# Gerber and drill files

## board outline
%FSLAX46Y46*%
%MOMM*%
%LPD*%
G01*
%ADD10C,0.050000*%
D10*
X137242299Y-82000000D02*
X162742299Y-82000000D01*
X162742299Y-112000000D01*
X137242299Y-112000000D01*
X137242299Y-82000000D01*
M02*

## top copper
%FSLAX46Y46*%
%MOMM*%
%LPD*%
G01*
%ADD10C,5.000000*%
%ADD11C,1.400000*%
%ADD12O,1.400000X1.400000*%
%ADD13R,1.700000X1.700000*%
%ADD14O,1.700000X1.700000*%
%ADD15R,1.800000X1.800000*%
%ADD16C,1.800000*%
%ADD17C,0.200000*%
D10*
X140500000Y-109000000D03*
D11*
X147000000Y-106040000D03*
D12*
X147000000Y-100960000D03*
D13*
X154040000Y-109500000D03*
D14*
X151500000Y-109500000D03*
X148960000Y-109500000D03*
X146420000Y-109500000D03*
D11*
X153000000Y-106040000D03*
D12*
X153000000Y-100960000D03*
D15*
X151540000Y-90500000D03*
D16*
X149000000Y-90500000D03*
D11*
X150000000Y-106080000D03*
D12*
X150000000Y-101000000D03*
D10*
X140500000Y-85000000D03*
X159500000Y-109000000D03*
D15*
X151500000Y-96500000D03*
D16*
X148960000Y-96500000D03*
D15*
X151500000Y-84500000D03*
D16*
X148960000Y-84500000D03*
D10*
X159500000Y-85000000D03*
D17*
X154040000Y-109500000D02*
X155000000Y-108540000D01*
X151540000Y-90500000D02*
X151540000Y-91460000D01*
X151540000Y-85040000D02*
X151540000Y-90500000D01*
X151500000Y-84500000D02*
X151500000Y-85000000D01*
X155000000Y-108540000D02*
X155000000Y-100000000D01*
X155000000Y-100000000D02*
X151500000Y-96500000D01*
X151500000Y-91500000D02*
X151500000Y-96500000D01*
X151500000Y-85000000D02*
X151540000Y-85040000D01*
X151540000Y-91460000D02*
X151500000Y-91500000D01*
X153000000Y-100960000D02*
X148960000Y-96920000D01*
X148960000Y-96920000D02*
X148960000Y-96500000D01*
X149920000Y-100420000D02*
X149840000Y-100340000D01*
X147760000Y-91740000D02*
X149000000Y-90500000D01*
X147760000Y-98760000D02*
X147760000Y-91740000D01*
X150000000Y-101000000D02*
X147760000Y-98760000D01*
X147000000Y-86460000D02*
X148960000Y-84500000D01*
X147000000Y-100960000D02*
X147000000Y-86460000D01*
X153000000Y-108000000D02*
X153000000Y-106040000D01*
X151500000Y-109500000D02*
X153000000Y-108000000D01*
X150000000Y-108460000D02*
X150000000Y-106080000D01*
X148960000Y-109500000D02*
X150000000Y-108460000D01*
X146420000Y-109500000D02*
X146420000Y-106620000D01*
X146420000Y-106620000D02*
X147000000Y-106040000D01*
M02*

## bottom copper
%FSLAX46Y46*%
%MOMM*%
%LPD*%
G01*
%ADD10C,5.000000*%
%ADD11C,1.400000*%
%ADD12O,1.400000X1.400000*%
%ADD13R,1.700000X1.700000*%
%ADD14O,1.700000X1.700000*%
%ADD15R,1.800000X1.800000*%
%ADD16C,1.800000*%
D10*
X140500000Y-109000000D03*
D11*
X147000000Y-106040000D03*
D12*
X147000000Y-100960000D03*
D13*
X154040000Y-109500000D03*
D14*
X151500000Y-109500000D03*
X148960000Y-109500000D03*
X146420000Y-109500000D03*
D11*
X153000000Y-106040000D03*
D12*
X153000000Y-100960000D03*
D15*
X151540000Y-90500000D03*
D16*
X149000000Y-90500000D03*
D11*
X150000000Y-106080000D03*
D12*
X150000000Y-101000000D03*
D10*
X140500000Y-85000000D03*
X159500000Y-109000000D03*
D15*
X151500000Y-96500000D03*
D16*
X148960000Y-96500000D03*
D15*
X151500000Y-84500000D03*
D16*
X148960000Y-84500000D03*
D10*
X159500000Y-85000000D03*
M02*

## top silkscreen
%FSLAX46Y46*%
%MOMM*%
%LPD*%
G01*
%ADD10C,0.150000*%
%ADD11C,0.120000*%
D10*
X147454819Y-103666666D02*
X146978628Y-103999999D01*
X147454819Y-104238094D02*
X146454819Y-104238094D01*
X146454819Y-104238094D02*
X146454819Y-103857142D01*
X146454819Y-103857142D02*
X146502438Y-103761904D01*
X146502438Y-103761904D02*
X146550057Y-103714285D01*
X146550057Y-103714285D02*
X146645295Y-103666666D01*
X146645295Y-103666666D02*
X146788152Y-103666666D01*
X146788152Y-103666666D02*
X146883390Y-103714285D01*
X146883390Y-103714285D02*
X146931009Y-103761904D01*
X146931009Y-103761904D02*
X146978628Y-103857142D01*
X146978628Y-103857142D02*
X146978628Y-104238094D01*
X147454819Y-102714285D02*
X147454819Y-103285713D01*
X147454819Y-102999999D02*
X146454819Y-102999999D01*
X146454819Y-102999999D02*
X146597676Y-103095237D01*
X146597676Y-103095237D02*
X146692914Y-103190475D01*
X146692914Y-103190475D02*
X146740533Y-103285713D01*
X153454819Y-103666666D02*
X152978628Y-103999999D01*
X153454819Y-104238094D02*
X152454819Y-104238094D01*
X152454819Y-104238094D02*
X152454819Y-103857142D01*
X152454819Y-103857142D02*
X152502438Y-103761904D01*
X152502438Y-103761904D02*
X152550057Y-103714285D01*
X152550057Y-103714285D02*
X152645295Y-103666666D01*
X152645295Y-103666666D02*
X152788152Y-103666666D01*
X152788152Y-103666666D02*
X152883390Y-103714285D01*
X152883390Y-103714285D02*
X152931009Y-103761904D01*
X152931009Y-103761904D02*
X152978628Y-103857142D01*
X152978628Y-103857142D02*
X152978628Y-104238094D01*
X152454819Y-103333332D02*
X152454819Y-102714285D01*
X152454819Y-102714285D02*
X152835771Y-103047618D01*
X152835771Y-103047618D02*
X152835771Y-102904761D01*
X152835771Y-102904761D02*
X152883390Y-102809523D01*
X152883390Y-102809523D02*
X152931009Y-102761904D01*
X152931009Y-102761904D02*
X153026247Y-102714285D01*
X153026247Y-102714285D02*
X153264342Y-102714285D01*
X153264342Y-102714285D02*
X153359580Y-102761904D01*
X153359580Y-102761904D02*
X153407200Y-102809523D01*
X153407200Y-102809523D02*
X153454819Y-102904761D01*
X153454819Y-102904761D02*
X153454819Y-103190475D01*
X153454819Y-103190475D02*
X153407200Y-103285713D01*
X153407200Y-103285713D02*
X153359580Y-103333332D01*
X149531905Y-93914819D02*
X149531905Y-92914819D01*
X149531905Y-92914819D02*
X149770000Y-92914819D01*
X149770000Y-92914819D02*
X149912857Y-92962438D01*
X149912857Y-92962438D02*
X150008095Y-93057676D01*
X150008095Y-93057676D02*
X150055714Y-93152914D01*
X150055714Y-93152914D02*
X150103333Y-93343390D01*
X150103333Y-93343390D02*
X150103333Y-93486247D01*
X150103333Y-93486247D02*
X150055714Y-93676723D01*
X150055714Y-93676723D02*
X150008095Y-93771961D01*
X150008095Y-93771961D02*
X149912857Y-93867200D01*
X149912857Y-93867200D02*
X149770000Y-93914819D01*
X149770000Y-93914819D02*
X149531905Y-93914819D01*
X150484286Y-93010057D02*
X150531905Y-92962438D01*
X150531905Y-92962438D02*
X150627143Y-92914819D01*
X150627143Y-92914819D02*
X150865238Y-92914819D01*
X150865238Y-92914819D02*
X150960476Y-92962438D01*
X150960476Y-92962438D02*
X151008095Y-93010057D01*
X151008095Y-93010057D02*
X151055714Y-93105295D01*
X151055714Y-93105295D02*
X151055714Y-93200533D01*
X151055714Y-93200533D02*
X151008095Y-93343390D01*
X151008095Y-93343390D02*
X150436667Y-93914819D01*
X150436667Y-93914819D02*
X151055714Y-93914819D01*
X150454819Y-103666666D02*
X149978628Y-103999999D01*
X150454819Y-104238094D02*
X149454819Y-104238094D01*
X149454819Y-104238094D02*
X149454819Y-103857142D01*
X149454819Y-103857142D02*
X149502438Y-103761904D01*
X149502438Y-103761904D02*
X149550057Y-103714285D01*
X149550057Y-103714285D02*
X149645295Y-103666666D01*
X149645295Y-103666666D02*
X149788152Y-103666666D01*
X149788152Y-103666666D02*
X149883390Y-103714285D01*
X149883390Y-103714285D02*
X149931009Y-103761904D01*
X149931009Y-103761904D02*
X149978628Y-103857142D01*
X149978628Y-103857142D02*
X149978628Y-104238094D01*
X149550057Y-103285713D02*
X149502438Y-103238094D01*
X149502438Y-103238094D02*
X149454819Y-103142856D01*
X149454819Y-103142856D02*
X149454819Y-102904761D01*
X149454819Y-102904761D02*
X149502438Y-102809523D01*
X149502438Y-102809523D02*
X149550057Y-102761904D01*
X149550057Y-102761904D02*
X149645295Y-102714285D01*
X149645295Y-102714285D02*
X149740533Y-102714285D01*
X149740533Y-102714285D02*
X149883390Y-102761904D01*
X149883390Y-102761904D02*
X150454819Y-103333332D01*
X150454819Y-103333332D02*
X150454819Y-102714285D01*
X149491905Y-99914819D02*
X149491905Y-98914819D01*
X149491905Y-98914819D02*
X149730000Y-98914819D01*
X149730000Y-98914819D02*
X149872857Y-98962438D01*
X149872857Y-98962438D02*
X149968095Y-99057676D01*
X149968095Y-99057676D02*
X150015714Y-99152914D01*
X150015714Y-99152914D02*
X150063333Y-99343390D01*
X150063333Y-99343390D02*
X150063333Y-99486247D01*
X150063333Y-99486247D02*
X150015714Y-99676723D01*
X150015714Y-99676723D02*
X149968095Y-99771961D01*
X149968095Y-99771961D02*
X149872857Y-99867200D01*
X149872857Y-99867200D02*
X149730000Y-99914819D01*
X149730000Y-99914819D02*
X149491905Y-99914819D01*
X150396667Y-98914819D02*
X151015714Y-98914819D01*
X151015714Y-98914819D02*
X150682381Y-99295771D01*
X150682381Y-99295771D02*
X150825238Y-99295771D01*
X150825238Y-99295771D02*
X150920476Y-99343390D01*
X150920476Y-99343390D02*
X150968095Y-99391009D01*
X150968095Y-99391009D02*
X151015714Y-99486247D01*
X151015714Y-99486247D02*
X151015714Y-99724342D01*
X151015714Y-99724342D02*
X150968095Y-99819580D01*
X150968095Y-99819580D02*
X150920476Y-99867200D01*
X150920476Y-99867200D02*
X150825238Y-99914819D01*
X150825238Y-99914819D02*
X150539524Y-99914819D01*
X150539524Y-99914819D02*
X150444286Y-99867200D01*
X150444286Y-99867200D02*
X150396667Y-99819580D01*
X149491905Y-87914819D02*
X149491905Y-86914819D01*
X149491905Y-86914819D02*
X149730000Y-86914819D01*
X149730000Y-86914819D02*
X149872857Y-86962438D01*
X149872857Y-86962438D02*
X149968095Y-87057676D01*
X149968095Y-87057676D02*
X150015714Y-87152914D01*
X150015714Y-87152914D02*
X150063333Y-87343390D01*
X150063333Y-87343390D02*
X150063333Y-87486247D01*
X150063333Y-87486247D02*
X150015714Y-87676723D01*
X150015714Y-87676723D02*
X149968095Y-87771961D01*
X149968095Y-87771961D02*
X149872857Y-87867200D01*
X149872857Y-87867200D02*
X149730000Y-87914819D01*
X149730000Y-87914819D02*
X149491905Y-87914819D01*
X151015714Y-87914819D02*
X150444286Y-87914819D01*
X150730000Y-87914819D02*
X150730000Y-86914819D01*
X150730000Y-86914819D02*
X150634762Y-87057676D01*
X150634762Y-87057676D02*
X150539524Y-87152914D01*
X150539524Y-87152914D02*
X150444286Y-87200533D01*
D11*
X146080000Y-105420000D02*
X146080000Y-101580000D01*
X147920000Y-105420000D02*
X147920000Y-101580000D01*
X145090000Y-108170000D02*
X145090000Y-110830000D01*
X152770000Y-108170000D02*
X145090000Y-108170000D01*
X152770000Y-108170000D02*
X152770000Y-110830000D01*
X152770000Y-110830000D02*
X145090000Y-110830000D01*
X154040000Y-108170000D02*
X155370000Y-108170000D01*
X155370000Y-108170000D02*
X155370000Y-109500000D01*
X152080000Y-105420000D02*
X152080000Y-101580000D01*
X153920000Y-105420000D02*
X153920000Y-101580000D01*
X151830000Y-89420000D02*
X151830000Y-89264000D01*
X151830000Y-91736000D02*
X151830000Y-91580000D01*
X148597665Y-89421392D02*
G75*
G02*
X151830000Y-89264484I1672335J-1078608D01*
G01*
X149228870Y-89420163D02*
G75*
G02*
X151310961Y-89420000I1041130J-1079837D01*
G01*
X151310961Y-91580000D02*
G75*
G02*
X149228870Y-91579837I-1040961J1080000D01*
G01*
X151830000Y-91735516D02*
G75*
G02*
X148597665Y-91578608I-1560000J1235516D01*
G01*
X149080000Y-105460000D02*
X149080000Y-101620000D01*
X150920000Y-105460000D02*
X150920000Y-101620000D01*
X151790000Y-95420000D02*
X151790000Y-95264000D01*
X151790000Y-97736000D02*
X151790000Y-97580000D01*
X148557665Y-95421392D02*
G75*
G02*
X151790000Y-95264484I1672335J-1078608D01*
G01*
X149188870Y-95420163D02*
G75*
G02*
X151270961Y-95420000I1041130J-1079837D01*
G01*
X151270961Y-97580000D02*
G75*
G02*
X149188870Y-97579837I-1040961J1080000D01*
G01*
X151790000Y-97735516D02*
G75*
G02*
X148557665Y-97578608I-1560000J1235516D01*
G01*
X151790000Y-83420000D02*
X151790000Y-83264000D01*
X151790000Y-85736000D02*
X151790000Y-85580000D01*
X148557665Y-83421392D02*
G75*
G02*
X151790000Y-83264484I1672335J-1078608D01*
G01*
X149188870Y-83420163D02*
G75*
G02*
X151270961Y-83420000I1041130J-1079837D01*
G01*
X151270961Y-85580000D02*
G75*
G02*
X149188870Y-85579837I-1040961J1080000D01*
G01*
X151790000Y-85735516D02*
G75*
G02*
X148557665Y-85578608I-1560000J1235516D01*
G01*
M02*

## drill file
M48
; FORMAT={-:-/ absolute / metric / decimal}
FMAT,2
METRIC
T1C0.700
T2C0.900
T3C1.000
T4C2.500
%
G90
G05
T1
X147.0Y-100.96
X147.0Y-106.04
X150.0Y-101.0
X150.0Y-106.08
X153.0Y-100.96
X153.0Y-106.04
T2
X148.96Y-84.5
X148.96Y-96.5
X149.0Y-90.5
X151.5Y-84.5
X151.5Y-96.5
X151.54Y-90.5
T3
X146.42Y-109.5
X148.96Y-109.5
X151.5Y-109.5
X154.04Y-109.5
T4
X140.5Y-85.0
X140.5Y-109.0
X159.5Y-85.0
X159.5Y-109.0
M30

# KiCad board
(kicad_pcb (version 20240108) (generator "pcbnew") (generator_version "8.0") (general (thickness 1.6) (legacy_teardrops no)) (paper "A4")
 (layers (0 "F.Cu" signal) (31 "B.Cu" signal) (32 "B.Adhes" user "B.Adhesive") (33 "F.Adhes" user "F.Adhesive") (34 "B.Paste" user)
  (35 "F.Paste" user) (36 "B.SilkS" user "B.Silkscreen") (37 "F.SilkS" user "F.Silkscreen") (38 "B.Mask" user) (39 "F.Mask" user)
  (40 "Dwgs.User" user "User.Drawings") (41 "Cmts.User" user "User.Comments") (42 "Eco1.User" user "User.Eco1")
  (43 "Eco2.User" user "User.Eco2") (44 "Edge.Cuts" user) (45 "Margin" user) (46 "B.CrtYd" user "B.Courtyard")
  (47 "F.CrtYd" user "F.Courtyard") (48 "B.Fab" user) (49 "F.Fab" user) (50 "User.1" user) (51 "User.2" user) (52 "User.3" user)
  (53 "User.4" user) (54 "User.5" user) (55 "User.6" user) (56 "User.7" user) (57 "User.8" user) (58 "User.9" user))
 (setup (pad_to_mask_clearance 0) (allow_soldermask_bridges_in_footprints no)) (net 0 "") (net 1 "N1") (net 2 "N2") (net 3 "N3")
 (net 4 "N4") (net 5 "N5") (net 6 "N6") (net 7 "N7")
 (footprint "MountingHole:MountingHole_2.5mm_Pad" (layer "F.Cu") (at 140.5 109)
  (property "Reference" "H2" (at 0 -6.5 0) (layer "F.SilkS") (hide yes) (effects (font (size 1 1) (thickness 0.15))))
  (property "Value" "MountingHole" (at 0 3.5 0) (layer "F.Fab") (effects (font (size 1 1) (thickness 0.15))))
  (pad "1" thru_hole circle (at 0 0) (size 5 5) (drill 2.5) (layers "*.Cu" "*.Mask") (remove_unused_layers no)))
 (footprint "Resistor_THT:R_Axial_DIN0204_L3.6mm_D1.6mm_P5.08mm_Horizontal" (layer "F.Cu") (at 147 106.04 90)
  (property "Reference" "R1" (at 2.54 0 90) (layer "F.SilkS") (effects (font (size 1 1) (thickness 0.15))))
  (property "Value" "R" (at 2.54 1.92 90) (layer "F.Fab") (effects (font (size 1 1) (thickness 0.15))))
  (fp_line (start 0.62 -0.92) (end 4.46 -0.92) (stroke (width 0.12) (type solid)) (layer "F.SilkS"))
  (fp_line (start 0.62 0.92) (end 4.46 0.92) (stroke (width 0.12) (type solid)) (layer "F.SilkS"))
  (pad "1" thru_hole circle (at 0 0 90) (size 1.4 1.4) (drill 0.7) (layers "*.Cu" "*.Mask") (remove_unused_layers no) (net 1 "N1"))
  (pad "2" thru_hole oval (at 5.08 0 90) (size 1.4 1.4) (drill 0.7) (layers "*.Cu" "*.Mask") (remove_unused_layers no) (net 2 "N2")))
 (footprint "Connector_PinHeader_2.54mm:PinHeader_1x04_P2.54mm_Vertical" (layer "F.Cu") (at 154.04 109.5 -90)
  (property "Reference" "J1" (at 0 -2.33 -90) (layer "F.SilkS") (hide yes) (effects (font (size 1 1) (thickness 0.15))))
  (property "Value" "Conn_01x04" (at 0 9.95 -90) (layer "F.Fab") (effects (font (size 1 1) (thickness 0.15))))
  (fp_line (start -1.33 8.95) (end 1.33 8.95) (stroke (width 0.12) (type solid)) (layer "F.SilkS"))
  (fp_line (start -1.33 1.27) (end -1.33 8.95) (stroke (width 0.12) (type solid)) (layer "F.SilkS"))
  (fp_line (start -1.33 1.27) (end 1.33 1.27) (stroke (width 0.12) (type solid)) (layer "F.SilkS"))
  (fp_line (start 1.33 1.27) (end 1.33 8.95) (stroke (width 0.12) (type solid)) (layer "F.SilkS"))
  (fp_line (start -1.33 0) (end -1.33 -1.33) (stroke (width 0.12) (type solid)) (layer "F.SilkS"))
  (fp_line (start -1.33 -1.33) (end 0 -1.33) (stroke (width 0.12) (type solid)) (layer "F.SilkS"))
  (pad "1" thru_hole rect (at 0 0 270) (size 1.7 1.7) (drill 1) (layers "*.Cu" "*.Mask") (remove_unused_layers no) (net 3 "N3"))
  (pad "2" thru_hole oval (at 0 2.54 270) (size 1.7 1.7) (drill 1) (layers "*.Cu" "*.Mask") (remove_unused_layers no) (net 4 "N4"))
  (pad "3" thru_hole oval (at 0 5.08 270) (size 1.7 1.7) (drill 1) (layers "*.Cu" "*.Mask") (remove_unused_layers no) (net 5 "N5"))
  (pad "4" thru_hole oval (at 0 7.62 270) (size 1.7 1.7) (drill 1) (layers "*.Cu" "*.Mask") (remove_unused_layers no) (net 1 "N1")))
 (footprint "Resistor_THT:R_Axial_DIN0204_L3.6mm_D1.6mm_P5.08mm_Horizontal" (layer "F.Cu") (at 153 106.04 90)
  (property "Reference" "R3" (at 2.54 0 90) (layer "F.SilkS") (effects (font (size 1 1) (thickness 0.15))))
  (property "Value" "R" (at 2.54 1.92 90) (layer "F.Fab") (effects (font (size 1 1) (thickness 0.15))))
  (fp_line (start 0.62 -0.92) (end 4.46 -0.92) (stroke (width 0.12) (type solid)) (layer "F.SilkS"))
  (fp_line (start 0.62 0.92) (end 4.46 0.92) (stroke (width 0.12) (type solid)) (layer "F.SilkS"))
  (pad "1" thru_hole circle (at 0 0 90) (size 1.4 1.4) (drill 0.7) (layers "*.Cu" "*.Mask") (remove_unused_layers no) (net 4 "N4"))
  (pad "2" thru_hole oval (at 5.08 0 90) (size 1.4 1.4) (drill 0.7) (layers "*.Cu" "*.Mask") (remove_unused_layers no) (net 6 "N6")))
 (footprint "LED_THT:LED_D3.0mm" (layer "F.Cu") (at 151.54 90.5 180)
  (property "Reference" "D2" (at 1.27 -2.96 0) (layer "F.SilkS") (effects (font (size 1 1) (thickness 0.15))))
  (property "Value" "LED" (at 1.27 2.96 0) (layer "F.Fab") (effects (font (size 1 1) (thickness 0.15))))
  (fp_line (start -0.29 1.08) (end -0.29 1.236) (stroke (width 0.12) (type solid)) (layer "F.SilkS"))
  (fp_line (start -0.29 -1.236) (end -0.29 -1.08) (stroke (width 0.12) (type solid)) (layer "F.SilkS"))
  (fp_arc (start 2.942335 1.078608) (mid 1.366487 1.987659) (end -0.29 1.235516) (stroke (width 0.12) (type solid)) (layer "F.SilkS"))
  (fp_arc (start 2.31113 1.079837) (mid 1.270117 1.5) (end 0.229039 1.08) (stroke (width 0.12) (type solid)) (layer "F.SilkS"))
  (fp_arc (start 0.229039 -1.08) (mid 1.270117 -1.5) (end 2.31113 -1.079837) (stroke (width 0.12) (type solid)) (layer "F.SilkS"))
  (fp_arc (start -0.29 -1.235516) (mid 1.366487 -1.987659) (end 2.942335 -1.078608) (stroke (width 0.12) (type solid)) (layer "F.SilkS"))
  (pad "1" thru_hole rect (at 0 0 180) (size 1.8 1.8) (drill 0.9) (layers "*.Cu" "*.Mask") (remove_unused_layers no) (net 3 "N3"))
  (pad "2" thru_hole circle (at 2.54 0 180) (size 1.8 1.8) (drill 0.9) (layers "*.Cu" "*.Mask") (remove_unused_layers no) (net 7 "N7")))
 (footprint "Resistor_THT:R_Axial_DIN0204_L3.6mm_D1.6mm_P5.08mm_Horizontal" (layer "F.Cu") (at 150 106.08 90)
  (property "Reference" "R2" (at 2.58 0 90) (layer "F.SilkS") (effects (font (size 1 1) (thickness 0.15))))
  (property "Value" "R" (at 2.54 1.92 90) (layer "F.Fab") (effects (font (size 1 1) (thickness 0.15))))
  (fp_line (start 0.62 -0.92) (end 4.46 -0.92) (stroke (width 0.12) (type solid)) (layer "F.SilkS"))
  (fp_line (start 0.62 0.92) (end 4.46 0.92) (stroke (width 0.12) (type solid)) (layer "F.SilkS"))
  (pad "1" thru_hole circle (at 0 0 90) (size 1.4 1.4) (drill 0.7) (layers "*.Cu" "*.Mask") (remove_unused_layers no) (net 5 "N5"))
  (pad "2" thru_hole oval (at 5.08 0 90) (size 1.4 1.4) (drill 0.7) (layers "*.Cu" "*.Mask") (remove_unused_layers no) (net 7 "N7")))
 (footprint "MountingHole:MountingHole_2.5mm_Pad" (layer "F.Cu") (at 140.5 85)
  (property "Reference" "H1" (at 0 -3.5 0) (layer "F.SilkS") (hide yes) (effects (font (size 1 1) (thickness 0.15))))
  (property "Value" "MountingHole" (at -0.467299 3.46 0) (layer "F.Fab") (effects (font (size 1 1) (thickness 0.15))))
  (pad "1" thru_hole circle (at 0 0) (size 5 5) (drill 2.5) (layers "*.Cu" "*.Mask") (remove_unused_layers no)))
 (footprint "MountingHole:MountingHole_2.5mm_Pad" (layer "F.Cu") (at 159.5 109)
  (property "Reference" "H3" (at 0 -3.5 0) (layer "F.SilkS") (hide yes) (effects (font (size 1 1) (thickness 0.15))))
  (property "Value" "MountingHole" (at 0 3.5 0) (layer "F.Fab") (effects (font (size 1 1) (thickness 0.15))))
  (pad "1" thru_hole circle (at 0 0) (size 5 5) (drill 2.5) (layers "*.Cu" "*.Mask") (remove_unused_layers no)))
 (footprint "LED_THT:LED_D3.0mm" (layer "F.Cu") (at 151.5 96.5 180)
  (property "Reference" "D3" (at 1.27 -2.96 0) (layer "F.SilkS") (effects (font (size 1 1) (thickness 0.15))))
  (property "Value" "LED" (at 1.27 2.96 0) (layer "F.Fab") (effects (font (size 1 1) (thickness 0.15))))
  (fp_line (start -0.29 1.08) (end -0.29 1.236) (stroke (width 0.12) (type solid)) (layer "F.SilkS"))
  (fp_line (start -0.29 -1.236) (end -0.29 -1.08) (stroke (width 0.12) (type solid)) (layer "F.SilkS"))
  (fp_arc (start 2.942335 1.078608) (mid 1.366487 1.987659) (end -0.29 1.235516) (stroke (width 0.12) (type solid)) (layer "F.SilkS"))
  (fp_arc (start 2.31113 1.079837) (mid 1.270117 1.5) (end 0.229039 1.08) (stroke (width 0.12) (type solid)) (layer "F.SilkS"))
  (fp_arc (start 0.229039 -1.08) (mid 1.270117 -1.5) (end 2.31113 -1.079837) (stroke (width 0.12) (type solid)) (layer "F.SilkS"))
  (fp_arc (start -0.29 -1.235516) (mid 1.366487 -1.987659) (end 2.942335 -1.078608) (stroke (width 0.12) (type solid)) (layer "F.SilkS"))
  (pad "1" thru_hole rect (at 0 0 180) (size 1.8 1.8) (drill 0.9) (layers "*.Cu" "*.Mask") (remove_unused_layers no) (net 3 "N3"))
  (pad "2" thru_hole circle (at 2.54 0 180) (size 1.8 1.8) (drill 0.9) (layers "*.Cu" "*.Mask") (remove_unused_layers no) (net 6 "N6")))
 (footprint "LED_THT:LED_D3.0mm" (layer "F.Cu") (at 151.5 84.5 180)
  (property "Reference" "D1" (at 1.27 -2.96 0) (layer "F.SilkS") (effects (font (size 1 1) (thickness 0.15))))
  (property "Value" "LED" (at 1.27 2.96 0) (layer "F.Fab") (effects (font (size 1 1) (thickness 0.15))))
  (fp_line (start -0.29 1.08) (end -0.29 1.236) (stroke (width 0.12) (type solid)) (layer "F.SilkS"))
  (fp_line (start -0.29 -1.236) (end -0.29 -1.08) (stroke (width 0.12) (type solid)) (layer "F.SilkS"))
  (fp_arc (start 2.942335 1.078608) (mid 1.366487 1.987659) (end -0.29 1.235516) (stroke (width 0.12) (type solid)) (layer "F.SilkS"))
  (fp_arc (start 2.31113 1.079837) (mid 1.270117 1.5) (end 0.229039 1.08) (stroke (width 0.12) (type solid)) (layer "F.SilkS"))
  (fp_arc (start 0.229039 -1.08) (mid 1.270117 -1.5) (end 2.31113 -1.079837) (stroke (width 0.12) (type solid)) (layer "F.SilkS"))
  (fp_arc (start -0.29 -1.235516) (mid 1.366487 -1.987659) (end 2.942335 -1.078608) (stroke (width 0.12) (type solid)) (layer "F.SilkS"))
  (pad "1" thru_hole rect (at 0 0 180) (size 1.8 1.8) (drill 0.9) (layers "*.Cu" "*.Mask") (remove_unused_layers no) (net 3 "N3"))
  (pad "2" thru_hole circle (at 2.54 0 180) (size 1.8 1.8) (drill 0.9) (layers "*.Cu" "*.Mask") (remove_unused_layers no) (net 2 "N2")))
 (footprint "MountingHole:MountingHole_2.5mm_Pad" (layer "F.Cu") (at 159.5 85)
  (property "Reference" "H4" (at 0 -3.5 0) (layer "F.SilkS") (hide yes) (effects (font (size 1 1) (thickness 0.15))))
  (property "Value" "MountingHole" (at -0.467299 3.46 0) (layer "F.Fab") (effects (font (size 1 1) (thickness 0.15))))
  (pad "1" thru_hole circle (at 0 0) (size 5 5) (drill 2.5) (layers "*.Cu" "*.Mask") (remove_unused_layers no)))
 (gr_rect (start 137.242299 82) (end 162.742299 112) (stroke (width 0.05) (type default)) (fill none) (layer "Edge.Cuts"))
 (segment (start 154.04 109.5) (end 155 108.54) (width 0.2) (layer "F.Cu") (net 3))
 (segment (start 151.54 90.5) (end 151.54 91.46) (width 0.2) (layer "F.Cu") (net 3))
 (segment (start 151.54 85.04) (end 151.54 90.5) (width 0.2) (layer "F.Cu") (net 3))
 (segment (start 151.5 84.5) (end 151.5 85) (width 0.2) (layer "F.Cu") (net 3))
 (segment (start 155 108.54) (end 155 100) (width 0.2) (layer "F.Cu") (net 3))
 (segment (start 155 100) (end 151.5 96.5) (width 0.2) (layer "F.Cu") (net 3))
 (segment (start 151.5 91.5) (end 151.5 96.5) (width 0.2) (layer "F.Cu") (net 3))
 (segment (start 151.5 85) (end 151.54 85.04) (width 0.2) (layer "F.Cu") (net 3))
 (segment (start 151.54 91.46) (end 151.5 91.5) (width 0.2) (layer "F.Cu") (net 3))
 (segment (start 153 100.96) (end 148.96 96.92) (width 0.2) (layer "F.Cu") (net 6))
 (segment (start 148.96 96.92) (end 148.96 96.5) (width 0.2) (layer "F.Cu") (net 6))
 (segment (start 149.92 100.42) (end 149.84 100.34) (width 0.2) (layer "F.Cu") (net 7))
 (segment (start 147.76 91.74) (end 149 90.5) (width 0.2) (layer "F.Cu") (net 7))
 (segment (start 147.76 98.76) (end 147.76 91.74) (width 0.2) (layer "F.Cu") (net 7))
 (segment (start 150 101) (end 147.76 98.76) (width 0.2) (layer "F.Cu") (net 7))
 (segment (start 147 86.46) (end 148.96 84.5) (width 0.2) (layer "F.Cu") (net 2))
 (segment (start 147 100.96) (end 147 86.46) (width 0.2) (layer "F.Cu") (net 2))
 (segment (start 153 108) (end 153 106.04) (width 0.2) (layer "F.Cu") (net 4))
 (segment (start 151.5 109.5) (end 153 108) (width 0.2) (layer "F.Cu") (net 4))
 (segment (start 150 108.46) (end 150 106.08) (width 0.2) (layer "F.Cu") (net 5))
 (segment (start 148.96 109.5) (end 150 108.46) (width 0.2) (layer "F.Cu") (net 5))
 (segment (start 146.42 109.5) (end 146.42 106.62) (width 0.2) (layer "F.Cu") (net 1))
 (segment (start 146.42 106.62) (end 147 106.04) (width 0.2) (layer "F.Cu") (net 1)))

